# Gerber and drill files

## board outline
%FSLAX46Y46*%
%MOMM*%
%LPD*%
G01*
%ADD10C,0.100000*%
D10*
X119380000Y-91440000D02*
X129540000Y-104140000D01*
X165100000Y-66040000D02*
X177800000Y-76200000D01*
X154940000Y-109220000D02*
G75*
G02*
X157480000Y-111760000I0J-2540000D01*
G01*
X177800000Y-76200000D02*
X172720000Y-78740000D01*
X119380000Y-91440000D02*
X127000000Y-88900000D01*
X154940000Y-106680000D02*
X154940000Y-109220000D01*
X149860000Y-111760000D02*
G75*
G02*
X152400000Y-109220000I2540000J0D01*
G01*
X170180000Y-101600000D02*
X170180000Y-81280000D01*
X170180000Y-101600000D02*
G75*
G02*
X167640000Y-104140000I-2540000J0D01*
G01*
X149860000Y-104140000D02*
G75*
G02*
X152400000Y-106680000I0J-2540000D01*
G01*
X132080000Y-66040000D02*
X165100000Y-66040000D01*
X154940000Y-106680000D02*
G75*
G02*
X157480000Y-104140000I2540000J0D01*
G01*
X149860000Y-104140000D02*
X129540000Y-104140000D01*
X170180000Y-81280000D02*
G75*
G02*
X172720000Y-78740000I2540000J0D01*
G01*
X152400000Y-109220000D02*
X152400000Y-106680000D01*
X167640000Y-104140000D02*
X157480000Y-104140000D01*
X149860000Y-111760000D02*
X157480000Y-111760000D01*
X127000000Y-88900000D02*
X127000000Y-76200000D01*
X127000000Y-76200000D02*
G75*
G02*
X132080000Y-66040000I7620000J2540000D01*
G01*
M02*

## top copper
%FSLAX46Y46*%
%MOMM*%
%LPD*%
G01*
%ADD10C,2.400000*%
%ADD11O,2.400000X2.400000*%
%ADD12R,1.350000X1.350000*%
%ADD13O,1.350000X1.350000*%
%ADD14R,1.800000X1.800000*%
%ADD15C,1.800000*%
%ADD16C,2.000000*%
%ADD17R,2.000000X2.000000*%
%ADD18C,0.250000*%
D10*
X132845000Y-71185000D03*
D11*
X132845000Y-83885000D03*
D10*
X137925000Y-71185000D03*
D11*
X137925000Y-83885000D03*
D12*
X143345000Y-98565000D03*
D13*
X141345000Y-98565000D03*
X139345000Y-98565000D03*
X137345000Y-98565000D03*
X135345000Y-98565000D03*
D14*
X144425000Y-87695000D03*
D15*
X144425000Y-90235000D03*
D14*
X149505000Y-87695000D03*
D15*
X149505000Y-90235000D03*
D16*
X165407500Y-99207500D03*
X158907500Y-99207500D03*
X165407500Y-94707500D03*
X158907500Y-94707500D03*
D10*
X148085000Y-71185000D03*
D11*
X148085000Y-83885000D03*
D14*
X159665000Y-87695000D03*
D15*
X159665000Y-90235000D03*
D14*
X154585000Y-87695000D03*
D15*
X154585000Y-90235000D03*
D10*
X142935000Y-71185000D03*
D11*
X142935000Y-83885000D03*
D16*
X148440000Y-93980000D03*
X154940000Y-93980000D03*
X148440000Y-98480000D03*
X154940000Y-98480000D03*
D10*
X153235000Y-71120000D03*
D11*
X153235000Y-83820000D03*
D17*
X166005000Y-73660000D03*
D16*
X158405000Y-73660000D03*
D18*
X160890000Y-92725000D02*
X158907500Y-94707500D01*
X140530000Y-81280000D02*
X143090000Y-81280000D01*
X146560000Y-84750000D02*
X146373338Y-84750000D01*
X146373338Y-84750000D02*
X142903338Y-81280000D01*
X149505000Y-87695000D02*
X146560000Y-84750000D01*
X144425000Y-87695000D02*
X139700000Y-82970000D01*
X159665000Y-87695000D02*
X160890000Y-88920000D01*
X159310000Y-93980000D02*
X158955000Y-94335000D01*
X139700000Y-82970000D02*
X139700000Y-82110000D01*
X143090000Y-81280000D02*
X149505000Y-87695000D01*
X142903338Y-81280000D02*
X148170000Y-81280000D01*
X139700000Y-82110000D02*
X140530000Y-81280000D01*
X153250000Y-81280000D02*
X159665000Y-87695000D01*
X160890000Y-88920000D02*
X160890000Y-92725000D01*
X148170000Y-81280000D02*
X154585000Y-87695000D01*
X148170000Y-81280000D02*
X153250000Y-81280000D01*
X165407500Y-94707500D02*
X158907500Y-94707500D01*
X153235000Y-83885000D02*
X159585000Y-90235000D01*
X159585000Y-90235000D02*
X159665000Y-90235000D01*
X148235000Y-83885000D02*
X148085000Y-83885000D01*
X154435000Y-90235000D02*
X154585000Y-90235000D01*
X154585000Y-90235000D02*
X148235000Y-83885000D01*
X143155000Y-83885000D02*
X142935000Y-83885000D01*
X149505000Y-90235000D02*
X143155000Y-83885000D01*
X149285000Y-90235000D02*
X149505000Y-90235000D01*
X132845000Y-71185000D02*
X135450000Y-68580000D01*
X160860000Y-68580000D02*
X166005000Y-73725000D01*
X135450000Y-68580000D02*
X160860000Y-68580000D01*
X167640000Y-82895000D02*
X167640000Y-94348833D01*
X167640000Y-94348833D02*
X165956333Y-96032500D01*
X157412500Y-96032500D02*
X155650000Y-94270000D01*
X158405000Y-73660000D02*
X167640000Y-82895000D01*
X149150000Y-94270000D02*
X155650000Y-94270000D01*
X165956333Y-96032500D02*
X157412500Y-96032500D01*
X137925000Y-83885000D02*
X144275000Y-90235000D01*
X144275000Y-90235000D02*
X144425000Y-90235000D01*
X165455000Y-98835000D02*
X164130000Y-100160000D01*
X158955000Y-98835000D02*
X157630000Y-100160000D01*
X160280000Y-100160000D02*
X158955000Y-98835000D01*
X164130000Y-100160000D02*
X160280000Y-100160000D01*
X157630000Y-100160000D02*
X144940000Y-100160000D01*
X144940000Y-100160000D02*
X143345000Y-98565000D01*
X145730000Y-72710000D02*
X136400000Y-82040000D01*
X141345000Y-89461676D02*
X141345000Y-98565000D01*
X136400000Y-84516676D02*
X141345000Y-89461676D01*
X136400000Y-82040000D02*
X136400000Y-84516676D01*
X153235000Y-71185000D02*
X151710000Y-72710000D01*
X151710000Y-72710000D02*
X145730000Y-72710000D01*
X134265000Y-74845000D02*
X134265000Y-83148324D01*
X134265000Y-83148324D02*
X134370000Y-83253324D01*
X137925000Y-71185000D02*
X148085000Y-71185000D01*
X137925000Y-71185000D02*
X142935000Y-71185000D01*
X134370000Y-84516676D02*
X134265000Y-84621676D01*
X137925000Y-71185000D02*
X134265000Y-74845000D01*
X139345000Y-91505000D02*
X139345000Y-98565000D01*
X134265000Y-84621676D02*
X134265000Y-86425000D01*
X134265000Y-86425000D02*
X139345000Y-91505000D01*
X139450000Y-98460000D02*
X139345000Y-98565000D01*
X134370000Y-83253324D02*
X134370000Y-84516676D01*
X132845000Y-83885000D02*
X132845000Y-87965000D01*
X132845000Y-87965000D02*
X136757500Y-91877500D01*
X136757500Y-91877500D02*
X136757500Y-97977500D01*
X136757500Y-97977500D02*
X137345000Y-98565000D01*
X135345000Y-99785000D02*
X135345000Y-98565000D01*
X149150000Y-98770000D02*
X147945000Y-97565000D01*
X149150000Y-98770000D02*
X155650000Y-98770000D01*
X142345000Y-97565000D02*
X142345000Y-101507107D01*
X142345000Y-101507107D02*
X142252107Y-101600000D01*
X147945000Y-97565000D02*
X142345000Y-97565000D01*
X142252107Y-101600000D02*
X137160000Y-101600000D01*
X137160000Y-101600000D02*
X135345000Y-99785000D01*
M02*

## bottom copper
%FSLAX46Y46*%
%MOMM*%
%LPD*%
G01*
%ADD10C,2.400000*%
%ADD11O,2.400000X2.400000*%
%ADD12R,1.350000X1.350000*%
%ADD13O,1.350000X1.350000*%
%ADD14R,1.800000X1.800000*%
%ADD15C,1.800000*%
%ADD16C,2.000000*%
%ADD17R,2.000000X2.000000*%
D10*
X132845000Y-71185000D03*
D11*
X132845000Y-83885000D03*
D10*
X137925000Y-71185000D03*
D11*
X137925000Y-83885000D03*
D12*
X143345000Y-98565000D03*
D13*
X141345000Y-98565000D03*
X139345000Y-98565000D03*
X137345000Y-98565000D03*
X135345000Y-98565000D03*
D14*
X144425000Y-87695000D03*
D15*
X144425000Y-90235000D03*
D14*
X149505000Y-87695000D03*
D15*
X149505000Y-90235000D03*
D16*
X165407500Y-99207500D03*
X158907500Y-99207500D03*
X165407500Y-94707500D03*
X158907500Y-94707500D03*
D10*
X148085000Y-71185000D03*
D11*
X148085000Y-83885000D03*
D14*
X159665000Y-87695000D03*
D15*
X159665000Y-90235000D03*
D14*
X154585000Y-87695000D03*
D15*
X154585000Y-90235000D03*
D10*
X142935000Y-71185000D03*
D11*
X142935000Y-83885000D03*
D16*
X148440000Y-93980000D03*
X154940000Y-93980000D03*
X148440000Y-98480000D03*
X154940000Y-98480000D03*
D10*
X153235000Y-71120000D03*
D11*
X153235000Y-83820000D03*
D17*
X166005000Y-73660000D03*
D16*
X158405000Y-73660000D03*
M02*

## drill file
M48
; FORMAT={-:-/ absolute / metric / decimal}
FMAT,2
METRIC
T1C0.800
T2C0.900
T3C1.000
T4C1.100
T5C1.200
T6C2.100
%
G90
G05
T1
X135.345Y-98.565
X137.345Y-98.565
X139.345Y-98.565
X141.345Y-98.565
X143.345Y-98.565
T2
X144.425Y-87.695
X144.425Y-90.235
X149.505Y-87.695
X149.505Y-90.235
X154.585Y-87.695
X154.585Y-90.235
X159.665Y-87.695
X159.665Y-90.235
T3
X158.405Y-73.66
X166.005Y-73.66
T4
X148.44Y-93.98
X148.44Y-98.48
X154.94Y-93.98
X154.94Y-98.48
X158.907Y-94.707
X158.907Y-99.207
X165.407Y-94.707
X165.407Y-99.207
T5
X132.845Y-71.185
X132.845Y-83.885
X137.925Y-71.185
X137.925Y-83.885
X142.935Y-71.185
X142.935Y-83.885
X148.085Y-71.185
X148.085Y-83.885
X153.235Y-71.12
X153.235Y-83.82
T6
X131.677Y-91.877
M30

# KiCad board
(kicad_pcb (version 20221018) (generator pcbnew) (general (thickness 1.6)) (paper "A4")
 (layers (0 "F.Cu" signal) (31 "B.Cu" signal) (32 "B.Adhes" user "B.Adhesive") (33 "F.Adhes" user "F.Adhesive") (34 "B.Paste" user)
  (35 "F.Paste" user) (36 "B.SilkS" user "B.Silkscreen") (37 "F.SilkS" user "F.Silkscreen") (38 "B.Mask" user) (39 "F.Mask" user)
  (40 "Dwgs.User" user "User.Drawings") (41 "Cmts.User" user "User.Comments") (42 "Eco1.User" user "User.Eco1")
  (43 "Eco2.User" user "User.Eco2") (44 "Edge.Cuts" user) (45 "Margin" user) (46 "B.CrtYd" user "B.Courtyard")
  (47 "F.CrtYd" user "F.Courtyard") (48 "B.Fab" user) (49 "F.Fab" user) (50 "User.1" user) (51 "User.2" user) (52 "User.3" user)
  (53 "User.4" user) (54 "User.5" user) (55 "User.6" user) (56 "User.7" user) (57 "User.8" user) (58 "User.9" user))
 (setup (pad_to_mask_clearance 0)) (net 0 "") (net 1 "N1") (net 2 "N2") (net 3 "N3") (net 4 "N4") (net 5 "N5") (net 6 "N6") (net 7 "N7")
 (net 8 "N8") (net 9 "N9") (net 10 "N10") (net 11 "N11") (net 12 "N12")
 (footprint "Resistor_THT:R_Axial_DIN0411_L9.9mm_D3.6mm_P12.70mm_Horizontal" (layer "F.Cu") (at 132.845 71.185 -90)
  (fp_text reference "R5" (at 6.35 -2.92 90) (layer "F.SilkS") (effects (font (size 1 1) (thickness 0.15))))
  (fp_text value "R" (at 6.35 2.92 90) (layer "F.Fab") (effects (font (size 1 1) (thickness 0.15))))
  (pad "1" thru_hole circle (at 0 0 270) (size 2.4 2.4) (drill 1.2) (layers "*.Cu" "*.Mask") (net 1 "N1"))
  (pad "2" thru_hole oval (at 12.7 0 270) (size 2.4 2.4) (drill 1.2) (layers "*.Cu" "*.Mask") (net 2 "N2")))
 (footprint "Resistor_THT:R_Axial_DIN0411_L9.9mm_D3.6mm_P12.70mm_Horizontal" (layer "F.Cu") (at 137.925 71.185 -90)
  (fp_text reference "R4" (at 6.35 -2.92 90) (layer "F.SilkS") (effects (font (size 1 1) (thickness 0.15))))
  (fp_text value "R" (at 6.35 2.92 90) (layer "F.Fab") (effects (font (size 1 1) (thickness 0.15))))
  (pad "1" thru_hole circle (at 0 0 270) (size 2.4 2.4) (drill 1.2) (layers "*.Cu" "*.Mask") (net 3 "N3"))
  (pad "2" thru_hole oval (at 12.7 0 270) (size 2.4 2.4) (drill 1.2) (layers "*.Cu" "*.Mask") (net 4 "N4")))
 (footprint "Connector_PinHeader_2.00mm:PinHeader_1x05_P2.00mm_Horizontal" (layer "F.Cu") (at 143.345 98.565 -90)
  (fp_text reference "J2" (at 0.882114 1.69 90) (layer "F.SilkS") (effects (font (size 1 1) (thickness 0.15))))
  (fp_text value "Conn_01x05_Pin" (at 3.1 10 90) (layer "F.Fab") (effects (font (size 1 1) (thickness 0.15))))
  (pad "1" thru_hole rect (at 0 0 270) (size 1.35 1.35) (drill 0.8) (layers "*.Cu" "*.Mask") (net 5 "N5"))
  (pad "2" thru_hole oval (at 0 2 270) (size 1.35 1.35) (drill 0.8) (layers "*.Cu" "*.Mask") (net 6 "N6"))
  (pad "3" thru_hole oval (at 0 4 270) (size 1.35 1.35) (drill 0.8) (layers "*.Cu" "*.Mask") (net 3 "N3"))
  (pad "4" thru_hole oval (at 0 6 270) (size 1.35 1.35) (drill 0.8) (layers "*.Cu" "*.Mask") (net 2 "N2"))
  (pad "5" thru_hole oval (at 0 8 270) (size 1.35 1.35) (drill 0.8) (layers "*.Cu" "*.Mask") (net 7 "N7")))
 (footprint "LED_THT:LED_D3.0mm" (layer "F.Cu") (at 144.425 87.695 -90)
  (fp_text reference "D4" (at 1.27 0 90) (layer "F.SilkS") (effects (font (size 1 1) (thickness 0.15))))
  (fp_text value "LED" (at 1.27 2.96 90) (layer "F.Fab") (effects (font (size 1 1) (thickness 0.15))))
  (pad "1" thru_hole rect (at 0 0 270) (size 1.8 1.8) (drill 0.9) (layers "*.Cu" "*.Mask") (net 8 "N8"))
  (pad "2" thru_hole circle (at 2.54 0 270) (size 1.8 1.8) (drill 0.9) (layers "*.Cu" "*.Mask") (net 4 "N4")))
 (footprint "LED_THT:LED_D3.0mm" (layer "F.Cu") (at 149.505 87.695 -90)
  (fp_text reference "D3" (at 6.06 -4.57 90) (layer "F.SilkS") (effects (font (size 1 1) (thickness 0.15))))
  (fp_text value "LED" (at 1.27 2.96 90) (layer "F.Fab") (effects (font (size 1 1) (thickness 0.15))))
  (pad "1" thru_hole rect (at 0 0 270) (size 1.8 1.8) (drill 0.9) (layers "*.Cu" "*.Mask") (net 8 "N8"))
  (pad "2" thru_hole circle (at 2.54 0 270) (size 1.8 1.8) (drill 0.9) (layers "*.Cu" "*.Mask") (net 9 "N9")))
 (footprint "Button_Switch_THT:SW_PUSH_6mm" (layer "F.Cu") (at 165.4075 99.2075 180)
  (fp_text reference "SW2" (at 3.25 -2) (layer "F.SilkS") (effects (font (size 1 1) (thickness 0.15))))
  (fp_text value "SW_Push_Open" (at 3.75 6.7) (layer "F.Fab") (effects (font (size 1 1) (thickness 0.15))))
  (pad "1" thru_hole circle (at 0 0 270) (size 2 2) (drill 1.1) (layers "*.Cu" "*.Mask") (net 5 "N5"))
  (pad "1" thru_hole circle (at 6.5 0 270) (size 2 2) (drill 1.1) (layers "*.Cu" "*.Mask") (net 5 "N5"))
  (pad "2" thru_hole circle (at 0 4.5 270) (size 2 2) (drill 1.1) (layers "*.Cu" "*.Mask") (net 8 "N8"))
  (pad "2" thru_hole circle (at 6.5 4.5 270) (size 2 2) (drill 1.1) (layers "*.Cu" "*.Mask") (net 8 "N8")))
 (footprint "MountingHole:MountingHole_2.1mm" (layer "F.Cu") (at 131.6775 91.8775 180)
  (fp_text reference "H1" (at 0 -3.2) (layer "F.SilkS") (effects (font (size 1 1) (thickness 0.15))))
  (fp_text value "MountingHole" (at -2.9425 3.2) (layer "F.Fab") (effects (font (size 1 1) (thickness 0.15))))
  (pad "" np_thru_hole circle (at 0 0 180) (size 2.1 2.1) (drill 2.1) (layers "*.Cu" "*.Mask")))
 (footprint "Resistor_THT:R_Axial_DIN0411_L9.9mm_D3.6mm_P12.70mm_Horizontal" (layer "F.Cu") (at 148.085 71.185 -90)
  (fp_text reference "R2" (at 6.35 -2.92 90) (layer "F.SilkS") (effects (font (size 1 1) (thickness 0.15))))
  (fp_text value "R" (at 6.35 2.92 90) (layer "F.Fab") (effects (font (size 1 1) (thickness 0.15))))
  (pad "1" thru_hole circle (at 0 0 270) (size 2.4 2.4) (drill 1.2) (layers "*.Cu" "*.Mask") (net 3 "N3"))
  (pad "2" thru_hole oval (at 12.7 0 270) (size 2.4 2.4) (drill 1.2) (layers "*.Cu" "*.Mask") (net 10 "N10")))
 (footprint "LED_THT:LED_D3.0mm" (layer "F.Cu") (at 159.665 87.695 -90)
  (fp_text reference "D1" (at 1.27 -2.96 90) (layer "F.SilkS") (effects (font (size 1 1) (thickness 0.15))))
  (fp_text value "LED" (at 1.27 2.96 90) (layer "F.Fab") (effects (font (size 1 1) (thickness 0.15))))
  (pad "1" thru_hole rect (at 0 0 270) (size 1.8 1.8) (drill 0.9) (layers "*.Cu" "*.Mask") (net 8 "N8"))
  (pad "2" thru_hole circle (at 2.54 0 270) (size 1.8 1.8) (drill 0.9) (layers "*.Cu" "*.Mask") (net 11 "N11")))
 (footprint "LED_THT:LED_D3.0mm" (layer "F.Cu") (at 154.585 87.695 -90)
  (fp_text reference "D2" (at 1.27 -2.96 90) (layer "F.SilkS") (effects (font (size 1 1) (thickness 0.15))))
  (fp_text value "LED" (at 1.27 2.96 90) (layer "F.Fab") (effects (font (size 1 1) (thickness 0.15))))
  (pad "1" thru_hole rect (at 0 0 270) (size 1.8 1.8) (drill 0.9) (layers "*.Cu" "*.Mask") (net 8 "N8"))
  (pad "2" thru_hole circle (at 2.54 0 270) (size 1.8 1.8) (drill 0.9) (layers "*.Cu" "*.Mask") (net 10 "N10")))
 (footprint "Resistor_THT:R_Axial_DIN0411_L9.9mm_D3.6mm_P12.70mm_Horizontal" (layer "F.Cu") (at 142.935 71.185 -90)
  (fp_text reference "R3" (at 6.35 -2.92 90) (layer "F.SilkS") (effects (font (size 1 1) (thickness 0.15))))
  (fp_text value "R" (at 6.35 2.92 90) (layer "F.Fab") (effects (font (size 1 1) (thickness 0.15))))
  (pad "1" thru_hole circle (at 0 0 270) (size 2.4 2.4) (drill 1.2) (layers "*.Cu" "*.Mask") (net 3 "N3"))
  (pad "2" thru_hole oval (at 12.7 0 270) (size 2.4 2.4) (drill 1.2) (layers "*.Cu" "*.Mask") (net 9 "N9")))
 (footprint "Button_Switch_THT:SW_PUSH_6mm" (layer "F.Cu") (at 148.44 93.98)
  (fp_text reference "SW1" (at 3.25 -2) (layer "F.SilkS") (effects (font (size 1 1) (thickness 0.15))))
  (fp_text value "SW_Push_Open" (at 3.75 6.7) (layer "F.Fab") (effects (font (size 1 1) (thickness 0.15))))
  (pad "1" thru_hole circle (at 0 0 90) (size 2 2) (drill 1.1) (layers "*.Cu" "*.Mask") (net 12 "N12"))
  (pad "1" thru_hole circle (at 6.5 0 90) (size 2 2) (drill 1.1) (layers "*.Cu" "*.Mask") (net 12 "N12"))
  (pad "2" thru_hole circle (at 0 4.5 90) (size 2 2) (drill 1.1) (layers "*.Cu" "*.Mask") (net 7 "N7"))
  (pad "2" thru_hole circle (at 6.5 4.5 90) (size 2 2) (drill 1.1) (layers "*.Cu" "*.Mask") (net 7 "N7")))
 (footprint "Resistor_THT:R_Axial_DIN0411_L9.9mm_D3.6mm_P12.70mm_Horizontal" (layer "F.Cu") (at 153.235 71.12 -90)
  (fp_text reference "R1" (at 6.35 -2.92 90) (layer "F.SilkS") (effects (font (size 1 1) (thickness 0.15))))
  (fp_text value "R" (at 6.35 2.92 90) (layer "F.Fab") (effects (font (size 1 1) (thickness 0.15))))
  (pad "1" thru_hole circle (at 0 0 270) (size 2.4 2.4) (drill 1.2) (layers "*.Cu" "*.Mask") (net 6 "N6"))
  (pad "2" thru_hole oval (at 12.7 0 270) (size 2.4 2.4) (drill 1.2) (layers "*.Cu" "*.Mask") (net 11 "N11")))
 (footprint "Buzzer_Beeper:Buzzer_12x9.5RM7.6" (layer "F.Cu") (at 166.005 73.66 180)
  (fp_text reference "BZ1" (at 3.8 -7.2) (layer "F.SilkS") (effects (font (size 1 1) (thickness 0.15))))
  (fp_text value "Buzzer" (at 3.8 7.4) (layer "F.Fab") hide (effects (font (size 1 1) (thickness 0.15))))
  (pad "1" thru_hole rect (at 0 0 180) (size 2 2) (drill 1) (layers "*.Cu" "*.Mask") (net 1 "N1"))
  (pad "2" thru_hole circle (at 7.6 0 180) (size 2 2) (drill 1) (layers "*.Cu" "*.Mask") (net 12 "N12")))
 (gr_line (start 119.38 91.44) (end 129.54 104.14) (stroke (width 0.1) (type default)) (layer "Edge.Cuts"))
 (gr_line (start 165.1 66.04) (end 177.8 76.2) (stroke (width 0.1) (type default)) (layer "Edge.Cuts"))
 (gr_arc (start 154.94 109.22) (mid 156.736051 109.963949) (end 157.48 111.76) (stroke (width 0.1) (type default)) (layer "Edge.Cuts"))
 (gr_line (start 177.8 76.2) (end 172.72 78.74) (stroke (width 0.1) (type default)) (layer "Edge.Cuts"))
 (gr_line (start 119.38 91.44) (end 127 88.9) (stroke (width 0.1) (type default)) (layer "Edge.Cuts"))
 (gr_line (start 154.94 106.68) (end 154.94 109.22) (stroke (width 0.1) (type default)) (layer "Edge.Cuts"))
 (gr_arc (start 149.86 111.76) (mid 150.603949 109.963949) (end 152.4 109.22) (stroke (width 0.1) (type default)) (layer "Edge.Cuts"))
 (gr_line (start 170.18 101.6) (end 170.18 81.28) (stroke (width 0.1) (type default)) (layer "Edge.Cuts"))
 (gr_arc (start 170.18 101.6) (mid 169.436051 103.396051) (end 167.64 104.14) (stroke (width 0.1) (type default)) (layer "Edge.Cuts"))
 (gr_arc (start 149.86 104.14) (mid 151.656051 104.883949) (end 152.4 106.68) (stroke (width 0.1) (type default)) (layer "Edge.Cuts"))
 (gr_line (start 132.08 66.04) (end 165.1 66.04) (stroke (width 0.1) (type default)) (layer "Edge.Cuts"))
 (gr_arc (start 154.94 106.68) (mid 155.683949 104.883949) (end 157.48 104.14) (stroke (width 0.1) (type default)) (layer "Edge.Cuts"))
 (gr_line (start 149.86 104.14) (end 129.54 104.14) (stroke (width 0.1) (type default)) (layer "Edge.Cuts"))
 (gr_arc (start 170.18 81.28) (mid 170.923949 79.483949) (end 172.72 78.74) (stroke (width 0.1) (type default)) (layer "Edge.Cuts"))
 (gr_line (start 152.4 109.22) (end 152.4 106.68) (stroke (width 0.1) (type default)) (layer "Edge.Cuts"))
 (gr_line (start 167.64 104.14) (end 157.48 104.14) (stroke (width 0.1) (type default)) (layer "Edge.Cuts"))
 (gr_line (start 149.86 111.76) (end 157.48 111.76) (stroke (width 0.1) (type default)) (layer "Edge.Cuts"))
 (gr_line (start 127 88.9) (end 127 76.2) (stroke (width 0.1) (type default)) (layer "Edge.Cuts"))
 (gr_arc (start 127 76.2) (mid 127.435795 70.067898) (end 132.08 66.04) (stroke (width 0.1) (type default)) (layer "Edge.Cuts"))
 (segment (start 160.89 92.725) (end 158.9075 94.7075) (width 0.25) (layer "F.Cu") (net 8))
 (segment (start 140.53 81.28) (end 143.09 81.28) (width 0.25) (layer "F.Cu") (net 8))
 (segment (start 146.56 84.75) (end 146.373338 84.75) (width 0.25) (layer "F.Cu") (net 8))
 (segment (start 146.373338 84.75) (end 142.903338 81.28) (width 0.25) (layer "F.Cu") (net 8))
 (segment (start 149.505 87.695) (end 146.56 84.75) (width 0.25) (layer "F.Cu") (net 8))
 (segment (start 144.425 87.695) (end 139.7 82.97) (width 0.25) (layer "F.Cu") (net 8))
 (segment (start 159.665 87.695) (end 160.89 88.92) (width 0.25) (layer "F.Cu") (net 8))
 (segment (start 159.31 93.98) (end 158.955 94.335) (width 0.25) (layer "F.Cu") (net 8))
 (segment (start 139.7 82.97) (end 139.7 82.11) (width 0.25) (layer "F.Cu") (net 8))
 (segment (start 143.09 81.28) (end 149.505 87.695) (width 0.25) (layer "F.Cu") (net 8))
 (segment (start 142.903338 81.28) (end 148.17 81.28) (width 0.25) (layer "F.Cu") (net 8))
 (segment (start 139.7 82.11) (end 140.53 81.28) (width 0.25) (layer "F.Cu") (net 8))
 (segment (start 153.25 81.28) (end 159.665 87.695) (width 0.25) (layer "F.Cu") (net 8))
 (segment (start 160.89 88.92) (end 160.89 92.725) (width 0.25) (layer "F.Cu") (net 8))
 (segment (start 148.17 81.28) (end 154.585 87.695) (width 0.25) (layer "F.Cu") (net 8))
 (segment (start 148.17 81.28) (end 153.25 81.28) (width 0.25) (layer "F.Cu") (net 8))
 (segment (start 165.4075 94.7075) (end 158.9075 94.7075) (width 0.25) (layer "F.Cu") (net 8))
 (segment (start 153.235 83.885) (end 159.585 90.235) (width 0.25) (layer "F.Cu") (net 11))
 (segment (start 159.585 90.235) (end 159.665 90.235) (width 0.25) (layer "F.Cu") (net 11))
 (segment (start 148.235 83.885) (end 148.085 83.885) (width 0.25) (layer "F.Cu") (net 10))
 (segment (start 154.435 90.235) (end 154.585 90.235) (width 0.25) (layer "F.Cu") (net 10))
 (segment (start 154.585 90.235) (end 148.235 83.885) (width 0.25) (layer "F.Cu") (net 10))
 (segment (start 143.155 83.885) (end 142.935 83.885) (width 0.25) (layer "F.Cu") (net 9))
 (segment (start 149.505 90.235) (end 143.155 83.885) (width 0.25) (layer "F.Cu") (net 9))
 (segment (start 149.285 90.235) (end 149.505 90.235) (width 0.25) (layer "F.Cu") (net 9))
 (segment (start 132.845 71.185) (end 135.45 68.58) (width 0.25) (layer "F.Cu") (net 1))
 (segment (start 160.86 68.58) (end 166.005 73.725) (width 0.25) (layer "F.Cu") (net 1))
 (segment (start 135.45 68.58) (end 160.86 68.58) (width 0.25) (layer "F.Cu") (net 1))
 (segment (start 167.64 82.895) (end 167.64 94.348833) (width 0.25) (layer "F.Cu") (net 12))
 (segment (start 167.64 94.348833) (end 165.956333 96.0325) (width 0.25) (layer "F.Cu") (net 12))
 (segment (start 157.4125 96.0325) (end 155.65 94.27) (width 0.25) (layer "F.Cu") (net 12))
 (segment (start 158.405 73.66) (end 167.64 82.895) (width 0.25) (layer "F.Cu") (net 12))
 (segment (start 149.15 94.27) (end 155.65 94.27) (width 0.25) (layer "F.Cu") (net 12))
 (segment (start 165.956333 96.0325) (end 157.4125 96.0325) (width 0.25) (layer "F.Cu") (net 12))
 (segment (start 137.925 83.885) (end 144.275 90.235) (width 0.25) (layer "F.Cu") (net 4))
 (segment (start 144.275 90.235) (end 144.425 90.235) (width 0.25) (layer "F.Cu") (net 4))
 (segment (start 165.455 98.835) (end 164.13 100.16) (width 0.25) (layer "F.Cu") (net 5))
 (segment (start 158.955 98.835) (end 157.63 100.16) (width 0.25) (layer "F.Cu") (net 5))
 (segment (start 160.28 100.16) (end 158.955 98.835) (width 0.25) (layer "F.Cu") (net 5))
 (segment (start 164.13 100.16) (end 160.28 100.16) (width 0.25) (layer "F.Cu") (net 5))
 (segment (start 157.63 100.16) (end 144.94 100.16) (width 0.25) (layer "F.Cu") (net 5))
 (segment (start 144.94 100.16) (end 143.345 98.565) (width 0.25) (layer "F.Cu") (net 5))
 (segment (start 145.73 72.71) (end 136.4 82.04) (width 0.25) (layer "F.Cu") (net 6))
 (segment (start 141.345 89.461676) (end 141.345 98.565) (width 0.25) (layer "F.Cu") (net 6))
 (segment (start 136.4 84.516676) (end 141.345 89.461676) (width 0.25) (layer "F.Cu") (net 6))
 (segment (start 136.4 82.04) (end 136.4 84.516676) (width 0.25) (layer "F.Cu") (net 6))
 (segment (start 153.235 71.185) (end 151.71 72.71) (width 0.25) (layer "F.Cu") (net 6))
 (segment (start 151.71 72.71) (end 145.73 72.71) (width 0.25) (layer "F.Cu") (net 6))
 (segment (start 134.265 74.845) (end 134.265 83.148324) (width 0.25) (layer "F.Cu") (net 3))
 (segment (start 134.265 83.148324) (end 134.37 83.253324) (width 0.25) (layer "F.Cu") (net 3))
 (segment (start 137.925 71.185) (end 148.085 71.185) (width 0.25) (layer "F.Cu") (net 3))
 (segment (start 137.925 71.185) (end 142.935 71.185) (width 0.25) (layer "F.Cu") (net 3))
 (segment (start 134.37 84.516676) (end 134.265 84.621676) (width 0.25) (layer "F.Cu") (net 3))
 (segment (start 137.925 71.185) (end 134.265 74.845) (width 0.25) (layer "F.Cu") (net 3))
 (segment (start 139.345 91.505) (end 139.345 98.565) (width 0.25) (layer "F.Cu") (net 3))
 (segment (start 134.265 84.621676) (end 134.265 86.425) (width 0.25) (layer "F.Cu") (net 3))
 (segment (start 134.265 86.425) (end 139.345 91.505) (width 0.25) (layer "F.Cu") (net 3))
 (segment (start 139.45 98.46) (end 139.345 98.565) (width 0.25) (layer "F.Cu") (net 3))
 (segment (start 134.37 83.253324) (end 134.37 84.516676) (width 0.25) (layer "F.Cu") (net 3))
 (segment (start 132.845 83.885) (end 132.845 87.965) (width 0.25) (layer "F.Cu") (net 2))
 (segment (start 132.845 87.965) (end 136.7575 91.8775) (width 0.25) (layer "F.Cu") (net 2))
 (segment (start 136.7575 91.8775) (end 136.7575 97.9775) (width 0.25) (layer "F.Cu") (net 2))
 (segment (start 136.7575 97.9775) (end 137.345 98.565) (width 0.25) (layer "F.Cu") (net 2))
 (segment (start 135.345 99.785) (end 135.345 98.565) (width 0.25) (layer "F.Cu") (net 7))
 (segment (start 149.15 98.77) (end 147.945 97.565) (width 0.25) (layer "F.Cu") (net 7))
 (segment (start 149.15 98.77) (end 155.65 98.77) (width 0.25) (layer "F.Cu") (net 7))
 (segment (start 142.345 97.565) (end 142.345 101.507107) (width 0.25) (layer "F.Cu") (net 7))
 (segment (start 142.345 101.507107) (end 142.252107 101.6) (width 0.25) (layer "F.Cu") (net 7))
 (segment (start 147.945 97.565) (end 142.345 97.565) (width 0.25) (layer "F.Cu") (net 7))
 (segment (start 142.252107 101.6) (end 137.16 101.6) (width 0.25) (layer "F.Cu") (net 7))
 (segment (start 137.16 101.6) (end 135.345 99.785) (width 0.25) (layer "F.Cu") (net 7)))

